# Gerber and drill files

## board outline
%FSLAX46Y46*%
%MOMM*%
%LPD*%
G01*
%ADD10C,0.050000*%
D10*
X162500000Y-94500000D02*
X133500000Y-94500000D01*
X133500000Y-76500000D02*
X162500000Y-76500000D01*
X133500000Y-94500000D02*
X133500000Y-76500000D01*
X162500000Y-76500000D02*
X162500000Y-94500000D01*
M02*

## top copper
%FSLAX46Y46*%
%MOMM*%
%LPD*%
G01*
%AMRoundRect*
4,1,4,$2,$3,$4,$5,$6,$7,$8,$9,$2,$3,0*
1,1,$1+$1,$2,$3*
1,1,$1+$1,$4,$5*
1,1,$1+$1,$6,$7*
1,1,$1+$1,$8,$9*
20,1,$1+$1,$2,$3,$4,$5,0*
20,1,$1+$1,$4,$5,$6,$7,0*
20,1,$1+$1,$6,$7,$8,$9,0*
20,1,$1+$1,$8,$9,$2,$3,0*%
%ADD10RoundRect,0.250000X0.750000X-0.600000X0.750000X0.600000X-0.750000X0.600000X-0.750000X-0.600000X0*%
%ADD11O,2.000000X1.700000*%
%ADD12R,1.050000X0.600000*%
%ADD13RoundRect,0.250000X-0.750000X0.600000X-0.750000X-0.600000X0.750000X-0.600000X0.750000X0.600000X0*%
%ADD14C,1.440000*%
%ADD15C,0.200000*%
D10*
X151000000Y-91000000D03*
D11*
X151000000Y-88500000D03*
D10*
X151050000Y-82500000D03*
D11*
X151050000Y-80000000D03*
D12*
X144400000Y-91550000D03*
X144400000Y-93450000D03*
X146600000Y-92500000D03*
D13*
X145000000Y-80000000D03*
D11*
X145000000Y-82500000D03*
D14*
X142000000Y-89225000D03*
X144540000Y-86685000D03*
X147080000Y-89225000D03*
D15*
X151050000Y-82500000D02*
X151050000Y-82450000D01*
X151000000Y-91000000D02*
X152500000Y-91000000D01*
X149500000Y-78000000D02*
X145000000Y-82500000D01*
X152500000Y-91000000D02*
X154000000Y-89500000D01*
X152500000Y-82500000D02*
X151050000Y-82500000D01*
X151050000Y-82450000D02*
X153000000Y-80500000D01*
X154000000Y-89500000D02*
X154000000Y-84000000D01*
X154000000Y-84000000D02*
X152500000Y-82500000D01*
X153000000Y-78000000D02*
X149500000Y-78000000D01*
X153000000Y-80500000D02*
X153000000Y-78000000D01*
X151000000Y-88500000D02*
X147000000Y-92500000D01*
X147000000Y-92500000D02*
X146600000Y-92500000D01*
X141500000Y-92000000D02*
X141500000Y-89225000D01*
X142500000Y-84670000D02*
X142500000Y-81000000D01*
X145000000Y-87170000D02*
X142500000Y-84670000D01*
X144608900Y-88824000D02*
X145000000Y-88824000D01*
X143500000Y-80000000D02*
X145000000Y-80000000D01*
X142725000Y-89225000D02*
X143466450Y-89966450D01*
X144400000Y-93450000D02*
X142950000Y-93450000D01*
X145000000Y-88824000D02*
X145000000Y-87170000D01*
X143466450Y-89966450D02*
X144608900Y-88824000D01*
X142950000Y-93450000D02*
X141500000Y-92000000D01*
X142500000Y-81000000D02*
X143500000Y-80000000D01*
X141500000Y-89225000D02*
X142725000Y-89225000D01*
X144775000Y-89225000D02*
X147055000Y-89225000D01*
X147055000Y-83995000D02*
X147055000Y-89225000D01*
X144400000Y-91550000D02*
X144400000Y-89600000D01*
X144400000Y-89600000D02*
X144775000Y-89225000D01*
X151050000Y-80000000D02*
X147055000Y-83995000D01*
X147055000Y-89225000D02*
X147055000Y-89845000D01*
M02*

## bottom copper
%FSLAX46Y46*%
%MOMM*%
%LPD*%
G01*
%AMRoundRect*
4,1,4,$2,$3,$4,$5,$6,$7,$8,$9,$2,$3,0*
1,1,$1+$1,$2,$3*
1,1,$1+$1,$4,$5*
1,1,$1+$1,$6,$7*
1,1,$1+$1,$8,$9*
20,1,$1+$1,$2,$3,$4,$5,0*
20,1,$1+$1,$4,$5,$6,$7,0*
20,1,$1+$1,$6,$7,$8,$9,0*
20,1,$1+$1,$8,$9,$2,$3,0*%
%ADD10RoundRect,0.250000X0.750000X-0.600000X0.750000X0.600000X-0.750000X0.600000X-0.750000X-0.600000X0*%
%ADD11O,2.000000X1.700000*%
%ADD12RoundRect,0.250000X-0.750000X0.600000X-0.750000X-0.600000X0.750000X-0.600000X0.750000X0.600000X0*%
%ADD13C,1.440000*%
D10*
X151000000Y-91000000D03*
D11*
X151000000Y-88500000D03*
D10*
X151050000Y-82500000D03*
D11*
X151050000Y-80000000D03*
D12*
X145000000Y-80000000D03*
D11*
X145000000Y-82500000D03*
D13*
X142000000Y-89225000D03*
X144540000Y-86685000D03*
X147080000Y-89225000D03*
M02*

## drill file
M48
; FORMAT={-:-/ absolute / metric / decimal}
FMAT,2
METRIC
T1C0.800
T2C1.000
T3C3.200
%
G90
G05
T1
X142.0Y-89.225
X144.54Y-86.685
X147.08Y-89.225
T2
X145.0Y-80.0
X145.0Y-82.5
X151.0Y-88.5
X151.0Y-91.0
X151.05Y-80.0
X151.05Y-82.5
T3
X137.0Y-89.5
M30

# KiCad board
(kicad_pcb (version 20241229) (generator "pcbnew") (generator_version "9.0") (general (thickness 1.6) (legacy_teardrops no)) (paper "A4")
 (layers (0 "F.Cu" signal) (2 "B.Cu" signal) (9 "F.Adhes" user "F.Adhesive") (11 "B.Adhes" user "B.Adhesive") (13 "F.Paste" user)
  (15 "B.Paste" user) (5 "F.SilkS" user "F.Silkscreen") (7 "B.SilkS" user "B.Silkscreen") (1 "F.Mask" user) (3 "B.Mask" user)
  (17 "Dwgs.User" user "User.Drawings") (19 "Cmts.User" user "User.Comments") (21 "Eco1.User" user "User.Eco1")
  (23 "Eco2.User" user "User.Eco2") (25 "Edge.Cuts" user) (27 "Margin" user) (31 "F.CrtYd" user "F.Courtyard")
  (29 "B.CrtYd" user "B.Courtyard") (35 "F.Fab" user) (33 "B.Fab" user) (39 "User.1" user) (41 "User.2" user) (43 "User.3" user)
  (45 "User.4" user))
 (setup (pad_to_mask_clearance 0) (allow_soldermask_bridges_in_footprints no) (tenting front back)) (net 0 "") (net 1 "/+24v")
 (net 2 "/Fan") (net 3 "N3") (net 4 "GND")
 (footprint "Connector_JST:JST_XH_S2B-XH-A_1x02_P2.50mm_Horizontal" (layer "F.Cu") (at 151 91 90)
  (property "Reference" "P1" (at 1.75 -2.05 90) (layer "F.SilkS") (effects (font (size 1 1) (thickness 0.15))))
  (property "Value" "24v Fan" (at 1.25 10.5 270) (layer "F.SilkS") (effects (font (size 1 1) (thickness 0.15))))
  (pad "1" thru_hole roundrect (at 0 0 90) (size 1.7 2) (drill 1) (layers "*.Cu" "*.Mask") (remove_unused_layers no)
   (roundrect_rratio 0.147059) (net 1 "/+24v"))
  (pad "2" thru_hole oval (at 2.5 0 90) (size 1.7 2) (drill 1) (layers "*.Cu" "*.Mask") (remove_unused_layers no) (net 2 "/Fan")))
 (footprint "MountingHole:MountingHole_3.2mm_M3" (layer "F.Cu") (at 137 89.5)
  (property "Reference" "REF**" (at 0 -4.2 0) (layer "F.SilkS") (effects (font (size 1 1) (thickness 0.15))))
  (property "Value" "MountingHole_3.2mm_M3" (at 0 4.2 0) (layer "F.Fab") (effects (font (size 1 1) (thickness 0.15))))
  (pad "" np_thru_hole circle (at 0 0) (size 3.2 3.2) (drill 3.2) (layers "*.Cu" "*.Mask")))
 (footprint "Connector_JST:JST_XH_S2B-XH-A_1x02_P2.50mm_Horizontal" (layer "F.Cu") (at 151.05 82.5 90)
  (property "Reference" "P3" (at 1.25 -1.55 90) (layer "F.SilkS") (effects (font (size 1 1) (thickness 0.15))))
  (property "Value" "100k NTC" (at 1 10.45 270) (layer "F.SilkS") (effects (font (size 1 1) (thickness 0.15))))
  (pad "1" thru_hole roundrect (at 0 0 90) (size 1.7 2) (drill 1) (layers "*.Cu" "*.Mask") (remove_unused_layers no)
   (roundrect_rratio 0.147059) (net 1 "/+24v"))
  (pad "2" thru_hole oval (at 2.5 0 90) (size 1.7 2) (drill 1) (layers "*.Cu" "*.Mask") (remove_unused_layers no) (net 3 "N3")))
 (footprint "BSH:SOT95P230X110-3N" (layer "F.Cu") (at 145.5 92.5)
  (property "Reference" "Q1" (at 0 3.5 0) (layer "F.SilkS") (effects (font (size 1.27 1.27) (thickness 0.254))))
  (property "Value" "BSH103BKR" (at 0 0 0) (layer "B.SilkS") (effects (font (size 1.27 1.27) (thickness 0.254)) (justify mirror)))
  (pad "1" smd rect (at -1.1 -0.95 90) (size 0.6 1.05) (layers "F.Cu" "F.Mask" "F.Paste") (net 3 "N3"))
  (pad "2" smd rect (at -1.1 0.95 90) (size 0.6 1.05) (layers "F.Cu" "F.Mask" "F.Paste") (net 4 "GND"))
  (pad "3" smd rect (at 1.1 0 90) (size 0.6 1.05) (layers "F.Cu" "F.Mask" "F.Paste") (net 2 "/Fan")))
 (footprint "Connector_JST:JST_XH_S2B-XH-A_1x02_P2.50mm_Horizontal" (layer "F.Cu") (at 145 80 -90)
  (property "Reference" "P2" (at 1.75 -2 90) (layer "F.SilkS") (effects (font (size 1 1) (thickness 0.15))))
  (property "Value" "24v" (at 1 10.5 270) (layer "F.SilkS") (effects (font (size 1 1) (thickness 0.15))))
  (pad "1" thru_hole roundrect (at 0 0 270) (size 1.7 2) (drill 1) (layers "*.Cu" "*.Mask") (remove_unused_layers no)
   (roundrect_rratio 0.147059) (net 4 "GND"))
  (pad "2" thru_hole oval (at 2.5 0 270) (size 1.7 2) (drill 1) (layers "*.Cu" "*.Mask") (remove_unused_layers no) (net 1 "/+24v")))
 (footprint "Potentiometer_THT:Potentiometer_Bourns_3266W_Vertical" (layer "F.Cu") (at 142 89.225 180)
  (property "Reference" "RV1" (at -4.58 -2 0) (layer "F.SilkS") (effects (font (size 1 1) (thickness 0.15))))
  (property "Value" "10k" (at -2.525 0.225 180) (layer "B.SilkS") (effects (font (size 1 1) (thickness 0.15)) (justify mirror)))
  (pad "1" thru_hole circle (at 0 0 180) (size 1.44 1.44) (drill 0.8) (layers "*.Cu" "*.Mask") (remove_unused_layers no) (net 4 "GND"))
  (pad "2" thru_hole circle (at -2.54 2.54 180) (size 1.44 1.44) (drill 0.8) (layers "*.Cu" "*.Mask") (remove_unused_layers no)
   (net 4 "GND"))
  (pad "3" thru_hole circle (at -5.08 0 180) (size 1.44 1.44) (drill 0.8) (layers "*.Cu" "*.Mask") (remove_unused_layers no) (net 3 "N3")))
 (gr_line (start 162.5 94.5) (end 133.5 94.5) (stroke (width 0.05) (type default)) (layer "Edge.Cuts"))
 (gr_line (start 133.5 76.5) (end 162.5 76.5) (stroke (width 0.05) (type default)) (layer "Edge.Cuts"))
 (gr_line (start 133.5 94.5) (end 133.5 76.5) (stroke (width 0.05) (type default)) (layer "Edge.Cuts"))
 (gr_line (start 162.5 76.5) (end 162.5 94.5) (stroke (width 0.05) (type default)) (layer "Edge.Cuts"))
 (segment (start 151.05 82.5) (end 151.05 82.45) (width 0.2) (layer "F.Cu") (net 1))
 (segment (start 151 91) (end 152.5 91) (width 0.2) (layer "F.Cu") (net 1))
 (segment (start 149.5 78) (end 145 82.5) (width 0.2) (layer "F.Cu") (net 1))
 (segment (start 152.5 91) (end 154 89.5) (width 0.2) (layer "F.Cu") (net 1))
 (segment (start 152.5 82.5) (end 151.05 82.5) (width 0.2) (layer "F.Cu") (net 1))
 (segment (start 151.05 82.45) (end 153 80.5) (width 0.2) (layer "F.Cu") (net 1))
 (segment (start 154 89.5) (end 154 84) (width 0.2) (layer "F.Cu") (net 1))
 (segment (start 154 84) (end 152.5 82.5) (width 0.2) (layer "F.Cu") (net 1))
 (segment (start 153 78) (end 149.5 78) (width 0.2) (layer "F.Cu") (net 1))
 (segment (start 153 80.5) (end 153 78) (width 0.2) (layer "F.Cu") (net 1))
 (segment (start 151 88.5) (end 147 92.5) (width 0.2) (layer "F.Cu") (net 2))
 (segment (start 147 92.5) (end 146.6 92.5) (width 0.2) (layer "F.Cu") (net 2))
 (segment (start 141.5 92) (end 141.5 89.225) (width 0.2) (layer "F.Cu") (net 4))
 (segment (start 142.5 84.67) (end 142.5 81) (width 0.2) (layer "F.Cu") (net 4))
 (segment (start 145 87.17) (end 142.5 84.67) (width 0.2) (layer "F.Cu") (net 4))
 (segment (start 144.6089 88.824) (end 145 88.824) (width 0.2) (layer "F.Cu") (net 4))
 (segment (start 143.5 80) (end 145 80) (width 0.2) (layer "F.Cu") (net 4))
 (segment (start 142.725 89.225) (end 143.46645 89.96645) (width 0.2) (layer "F.Cu") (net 4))
 (segment (start 144.4 93.45) (end 142.95 93.45) (width 0.2) (layer "F.Cu") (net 4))
 (segment (start 145 88.824) (end 145 87.17) (width 0.2) (layer "F.Cu") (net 4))
 (segment (start 143.46645 89.96645) (end 144.6089 88.824) (width 0.2) (layer "F.Cu") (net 4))
 (segment (start 142.95 93.45) (end 141.5 92) (width 0.2) (layer "F.Cu") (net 4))
 (segment (start 142.5 81) (end 143.5 80) (width 0.2) (layer "F.Cu") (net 4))
 (segment (start 141.5 89.225) (end 142.725 89.225) (width 0.2) (layer "F.Cu") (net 4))
 (segment (start 144.775 89.225) (end 147.055 89.225) (width 0.2) (layer "F.Cu") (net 3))
 (segment (start 147.055 83.995) (end 147.055 89.225) (width 0.2) (layer "F.Cu") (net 3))
 (segment (start 144.4 91.55) (end 144.4 89.6) (width 0.2) (layer "F.Cu") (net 3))
 (segment (start 144.4 89.6) (end 144.775 89.225) (width 0.2) (layer "F.Cu") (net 3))
 (segment (start 151.05 80) (end 147.055 83.995) (width 0.2) (layer "F.Cu") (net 3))
 (segment (start 147.055 89.225) (end 147.055 89.845) (width 0.2) (layer "F.Cu") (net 3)))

